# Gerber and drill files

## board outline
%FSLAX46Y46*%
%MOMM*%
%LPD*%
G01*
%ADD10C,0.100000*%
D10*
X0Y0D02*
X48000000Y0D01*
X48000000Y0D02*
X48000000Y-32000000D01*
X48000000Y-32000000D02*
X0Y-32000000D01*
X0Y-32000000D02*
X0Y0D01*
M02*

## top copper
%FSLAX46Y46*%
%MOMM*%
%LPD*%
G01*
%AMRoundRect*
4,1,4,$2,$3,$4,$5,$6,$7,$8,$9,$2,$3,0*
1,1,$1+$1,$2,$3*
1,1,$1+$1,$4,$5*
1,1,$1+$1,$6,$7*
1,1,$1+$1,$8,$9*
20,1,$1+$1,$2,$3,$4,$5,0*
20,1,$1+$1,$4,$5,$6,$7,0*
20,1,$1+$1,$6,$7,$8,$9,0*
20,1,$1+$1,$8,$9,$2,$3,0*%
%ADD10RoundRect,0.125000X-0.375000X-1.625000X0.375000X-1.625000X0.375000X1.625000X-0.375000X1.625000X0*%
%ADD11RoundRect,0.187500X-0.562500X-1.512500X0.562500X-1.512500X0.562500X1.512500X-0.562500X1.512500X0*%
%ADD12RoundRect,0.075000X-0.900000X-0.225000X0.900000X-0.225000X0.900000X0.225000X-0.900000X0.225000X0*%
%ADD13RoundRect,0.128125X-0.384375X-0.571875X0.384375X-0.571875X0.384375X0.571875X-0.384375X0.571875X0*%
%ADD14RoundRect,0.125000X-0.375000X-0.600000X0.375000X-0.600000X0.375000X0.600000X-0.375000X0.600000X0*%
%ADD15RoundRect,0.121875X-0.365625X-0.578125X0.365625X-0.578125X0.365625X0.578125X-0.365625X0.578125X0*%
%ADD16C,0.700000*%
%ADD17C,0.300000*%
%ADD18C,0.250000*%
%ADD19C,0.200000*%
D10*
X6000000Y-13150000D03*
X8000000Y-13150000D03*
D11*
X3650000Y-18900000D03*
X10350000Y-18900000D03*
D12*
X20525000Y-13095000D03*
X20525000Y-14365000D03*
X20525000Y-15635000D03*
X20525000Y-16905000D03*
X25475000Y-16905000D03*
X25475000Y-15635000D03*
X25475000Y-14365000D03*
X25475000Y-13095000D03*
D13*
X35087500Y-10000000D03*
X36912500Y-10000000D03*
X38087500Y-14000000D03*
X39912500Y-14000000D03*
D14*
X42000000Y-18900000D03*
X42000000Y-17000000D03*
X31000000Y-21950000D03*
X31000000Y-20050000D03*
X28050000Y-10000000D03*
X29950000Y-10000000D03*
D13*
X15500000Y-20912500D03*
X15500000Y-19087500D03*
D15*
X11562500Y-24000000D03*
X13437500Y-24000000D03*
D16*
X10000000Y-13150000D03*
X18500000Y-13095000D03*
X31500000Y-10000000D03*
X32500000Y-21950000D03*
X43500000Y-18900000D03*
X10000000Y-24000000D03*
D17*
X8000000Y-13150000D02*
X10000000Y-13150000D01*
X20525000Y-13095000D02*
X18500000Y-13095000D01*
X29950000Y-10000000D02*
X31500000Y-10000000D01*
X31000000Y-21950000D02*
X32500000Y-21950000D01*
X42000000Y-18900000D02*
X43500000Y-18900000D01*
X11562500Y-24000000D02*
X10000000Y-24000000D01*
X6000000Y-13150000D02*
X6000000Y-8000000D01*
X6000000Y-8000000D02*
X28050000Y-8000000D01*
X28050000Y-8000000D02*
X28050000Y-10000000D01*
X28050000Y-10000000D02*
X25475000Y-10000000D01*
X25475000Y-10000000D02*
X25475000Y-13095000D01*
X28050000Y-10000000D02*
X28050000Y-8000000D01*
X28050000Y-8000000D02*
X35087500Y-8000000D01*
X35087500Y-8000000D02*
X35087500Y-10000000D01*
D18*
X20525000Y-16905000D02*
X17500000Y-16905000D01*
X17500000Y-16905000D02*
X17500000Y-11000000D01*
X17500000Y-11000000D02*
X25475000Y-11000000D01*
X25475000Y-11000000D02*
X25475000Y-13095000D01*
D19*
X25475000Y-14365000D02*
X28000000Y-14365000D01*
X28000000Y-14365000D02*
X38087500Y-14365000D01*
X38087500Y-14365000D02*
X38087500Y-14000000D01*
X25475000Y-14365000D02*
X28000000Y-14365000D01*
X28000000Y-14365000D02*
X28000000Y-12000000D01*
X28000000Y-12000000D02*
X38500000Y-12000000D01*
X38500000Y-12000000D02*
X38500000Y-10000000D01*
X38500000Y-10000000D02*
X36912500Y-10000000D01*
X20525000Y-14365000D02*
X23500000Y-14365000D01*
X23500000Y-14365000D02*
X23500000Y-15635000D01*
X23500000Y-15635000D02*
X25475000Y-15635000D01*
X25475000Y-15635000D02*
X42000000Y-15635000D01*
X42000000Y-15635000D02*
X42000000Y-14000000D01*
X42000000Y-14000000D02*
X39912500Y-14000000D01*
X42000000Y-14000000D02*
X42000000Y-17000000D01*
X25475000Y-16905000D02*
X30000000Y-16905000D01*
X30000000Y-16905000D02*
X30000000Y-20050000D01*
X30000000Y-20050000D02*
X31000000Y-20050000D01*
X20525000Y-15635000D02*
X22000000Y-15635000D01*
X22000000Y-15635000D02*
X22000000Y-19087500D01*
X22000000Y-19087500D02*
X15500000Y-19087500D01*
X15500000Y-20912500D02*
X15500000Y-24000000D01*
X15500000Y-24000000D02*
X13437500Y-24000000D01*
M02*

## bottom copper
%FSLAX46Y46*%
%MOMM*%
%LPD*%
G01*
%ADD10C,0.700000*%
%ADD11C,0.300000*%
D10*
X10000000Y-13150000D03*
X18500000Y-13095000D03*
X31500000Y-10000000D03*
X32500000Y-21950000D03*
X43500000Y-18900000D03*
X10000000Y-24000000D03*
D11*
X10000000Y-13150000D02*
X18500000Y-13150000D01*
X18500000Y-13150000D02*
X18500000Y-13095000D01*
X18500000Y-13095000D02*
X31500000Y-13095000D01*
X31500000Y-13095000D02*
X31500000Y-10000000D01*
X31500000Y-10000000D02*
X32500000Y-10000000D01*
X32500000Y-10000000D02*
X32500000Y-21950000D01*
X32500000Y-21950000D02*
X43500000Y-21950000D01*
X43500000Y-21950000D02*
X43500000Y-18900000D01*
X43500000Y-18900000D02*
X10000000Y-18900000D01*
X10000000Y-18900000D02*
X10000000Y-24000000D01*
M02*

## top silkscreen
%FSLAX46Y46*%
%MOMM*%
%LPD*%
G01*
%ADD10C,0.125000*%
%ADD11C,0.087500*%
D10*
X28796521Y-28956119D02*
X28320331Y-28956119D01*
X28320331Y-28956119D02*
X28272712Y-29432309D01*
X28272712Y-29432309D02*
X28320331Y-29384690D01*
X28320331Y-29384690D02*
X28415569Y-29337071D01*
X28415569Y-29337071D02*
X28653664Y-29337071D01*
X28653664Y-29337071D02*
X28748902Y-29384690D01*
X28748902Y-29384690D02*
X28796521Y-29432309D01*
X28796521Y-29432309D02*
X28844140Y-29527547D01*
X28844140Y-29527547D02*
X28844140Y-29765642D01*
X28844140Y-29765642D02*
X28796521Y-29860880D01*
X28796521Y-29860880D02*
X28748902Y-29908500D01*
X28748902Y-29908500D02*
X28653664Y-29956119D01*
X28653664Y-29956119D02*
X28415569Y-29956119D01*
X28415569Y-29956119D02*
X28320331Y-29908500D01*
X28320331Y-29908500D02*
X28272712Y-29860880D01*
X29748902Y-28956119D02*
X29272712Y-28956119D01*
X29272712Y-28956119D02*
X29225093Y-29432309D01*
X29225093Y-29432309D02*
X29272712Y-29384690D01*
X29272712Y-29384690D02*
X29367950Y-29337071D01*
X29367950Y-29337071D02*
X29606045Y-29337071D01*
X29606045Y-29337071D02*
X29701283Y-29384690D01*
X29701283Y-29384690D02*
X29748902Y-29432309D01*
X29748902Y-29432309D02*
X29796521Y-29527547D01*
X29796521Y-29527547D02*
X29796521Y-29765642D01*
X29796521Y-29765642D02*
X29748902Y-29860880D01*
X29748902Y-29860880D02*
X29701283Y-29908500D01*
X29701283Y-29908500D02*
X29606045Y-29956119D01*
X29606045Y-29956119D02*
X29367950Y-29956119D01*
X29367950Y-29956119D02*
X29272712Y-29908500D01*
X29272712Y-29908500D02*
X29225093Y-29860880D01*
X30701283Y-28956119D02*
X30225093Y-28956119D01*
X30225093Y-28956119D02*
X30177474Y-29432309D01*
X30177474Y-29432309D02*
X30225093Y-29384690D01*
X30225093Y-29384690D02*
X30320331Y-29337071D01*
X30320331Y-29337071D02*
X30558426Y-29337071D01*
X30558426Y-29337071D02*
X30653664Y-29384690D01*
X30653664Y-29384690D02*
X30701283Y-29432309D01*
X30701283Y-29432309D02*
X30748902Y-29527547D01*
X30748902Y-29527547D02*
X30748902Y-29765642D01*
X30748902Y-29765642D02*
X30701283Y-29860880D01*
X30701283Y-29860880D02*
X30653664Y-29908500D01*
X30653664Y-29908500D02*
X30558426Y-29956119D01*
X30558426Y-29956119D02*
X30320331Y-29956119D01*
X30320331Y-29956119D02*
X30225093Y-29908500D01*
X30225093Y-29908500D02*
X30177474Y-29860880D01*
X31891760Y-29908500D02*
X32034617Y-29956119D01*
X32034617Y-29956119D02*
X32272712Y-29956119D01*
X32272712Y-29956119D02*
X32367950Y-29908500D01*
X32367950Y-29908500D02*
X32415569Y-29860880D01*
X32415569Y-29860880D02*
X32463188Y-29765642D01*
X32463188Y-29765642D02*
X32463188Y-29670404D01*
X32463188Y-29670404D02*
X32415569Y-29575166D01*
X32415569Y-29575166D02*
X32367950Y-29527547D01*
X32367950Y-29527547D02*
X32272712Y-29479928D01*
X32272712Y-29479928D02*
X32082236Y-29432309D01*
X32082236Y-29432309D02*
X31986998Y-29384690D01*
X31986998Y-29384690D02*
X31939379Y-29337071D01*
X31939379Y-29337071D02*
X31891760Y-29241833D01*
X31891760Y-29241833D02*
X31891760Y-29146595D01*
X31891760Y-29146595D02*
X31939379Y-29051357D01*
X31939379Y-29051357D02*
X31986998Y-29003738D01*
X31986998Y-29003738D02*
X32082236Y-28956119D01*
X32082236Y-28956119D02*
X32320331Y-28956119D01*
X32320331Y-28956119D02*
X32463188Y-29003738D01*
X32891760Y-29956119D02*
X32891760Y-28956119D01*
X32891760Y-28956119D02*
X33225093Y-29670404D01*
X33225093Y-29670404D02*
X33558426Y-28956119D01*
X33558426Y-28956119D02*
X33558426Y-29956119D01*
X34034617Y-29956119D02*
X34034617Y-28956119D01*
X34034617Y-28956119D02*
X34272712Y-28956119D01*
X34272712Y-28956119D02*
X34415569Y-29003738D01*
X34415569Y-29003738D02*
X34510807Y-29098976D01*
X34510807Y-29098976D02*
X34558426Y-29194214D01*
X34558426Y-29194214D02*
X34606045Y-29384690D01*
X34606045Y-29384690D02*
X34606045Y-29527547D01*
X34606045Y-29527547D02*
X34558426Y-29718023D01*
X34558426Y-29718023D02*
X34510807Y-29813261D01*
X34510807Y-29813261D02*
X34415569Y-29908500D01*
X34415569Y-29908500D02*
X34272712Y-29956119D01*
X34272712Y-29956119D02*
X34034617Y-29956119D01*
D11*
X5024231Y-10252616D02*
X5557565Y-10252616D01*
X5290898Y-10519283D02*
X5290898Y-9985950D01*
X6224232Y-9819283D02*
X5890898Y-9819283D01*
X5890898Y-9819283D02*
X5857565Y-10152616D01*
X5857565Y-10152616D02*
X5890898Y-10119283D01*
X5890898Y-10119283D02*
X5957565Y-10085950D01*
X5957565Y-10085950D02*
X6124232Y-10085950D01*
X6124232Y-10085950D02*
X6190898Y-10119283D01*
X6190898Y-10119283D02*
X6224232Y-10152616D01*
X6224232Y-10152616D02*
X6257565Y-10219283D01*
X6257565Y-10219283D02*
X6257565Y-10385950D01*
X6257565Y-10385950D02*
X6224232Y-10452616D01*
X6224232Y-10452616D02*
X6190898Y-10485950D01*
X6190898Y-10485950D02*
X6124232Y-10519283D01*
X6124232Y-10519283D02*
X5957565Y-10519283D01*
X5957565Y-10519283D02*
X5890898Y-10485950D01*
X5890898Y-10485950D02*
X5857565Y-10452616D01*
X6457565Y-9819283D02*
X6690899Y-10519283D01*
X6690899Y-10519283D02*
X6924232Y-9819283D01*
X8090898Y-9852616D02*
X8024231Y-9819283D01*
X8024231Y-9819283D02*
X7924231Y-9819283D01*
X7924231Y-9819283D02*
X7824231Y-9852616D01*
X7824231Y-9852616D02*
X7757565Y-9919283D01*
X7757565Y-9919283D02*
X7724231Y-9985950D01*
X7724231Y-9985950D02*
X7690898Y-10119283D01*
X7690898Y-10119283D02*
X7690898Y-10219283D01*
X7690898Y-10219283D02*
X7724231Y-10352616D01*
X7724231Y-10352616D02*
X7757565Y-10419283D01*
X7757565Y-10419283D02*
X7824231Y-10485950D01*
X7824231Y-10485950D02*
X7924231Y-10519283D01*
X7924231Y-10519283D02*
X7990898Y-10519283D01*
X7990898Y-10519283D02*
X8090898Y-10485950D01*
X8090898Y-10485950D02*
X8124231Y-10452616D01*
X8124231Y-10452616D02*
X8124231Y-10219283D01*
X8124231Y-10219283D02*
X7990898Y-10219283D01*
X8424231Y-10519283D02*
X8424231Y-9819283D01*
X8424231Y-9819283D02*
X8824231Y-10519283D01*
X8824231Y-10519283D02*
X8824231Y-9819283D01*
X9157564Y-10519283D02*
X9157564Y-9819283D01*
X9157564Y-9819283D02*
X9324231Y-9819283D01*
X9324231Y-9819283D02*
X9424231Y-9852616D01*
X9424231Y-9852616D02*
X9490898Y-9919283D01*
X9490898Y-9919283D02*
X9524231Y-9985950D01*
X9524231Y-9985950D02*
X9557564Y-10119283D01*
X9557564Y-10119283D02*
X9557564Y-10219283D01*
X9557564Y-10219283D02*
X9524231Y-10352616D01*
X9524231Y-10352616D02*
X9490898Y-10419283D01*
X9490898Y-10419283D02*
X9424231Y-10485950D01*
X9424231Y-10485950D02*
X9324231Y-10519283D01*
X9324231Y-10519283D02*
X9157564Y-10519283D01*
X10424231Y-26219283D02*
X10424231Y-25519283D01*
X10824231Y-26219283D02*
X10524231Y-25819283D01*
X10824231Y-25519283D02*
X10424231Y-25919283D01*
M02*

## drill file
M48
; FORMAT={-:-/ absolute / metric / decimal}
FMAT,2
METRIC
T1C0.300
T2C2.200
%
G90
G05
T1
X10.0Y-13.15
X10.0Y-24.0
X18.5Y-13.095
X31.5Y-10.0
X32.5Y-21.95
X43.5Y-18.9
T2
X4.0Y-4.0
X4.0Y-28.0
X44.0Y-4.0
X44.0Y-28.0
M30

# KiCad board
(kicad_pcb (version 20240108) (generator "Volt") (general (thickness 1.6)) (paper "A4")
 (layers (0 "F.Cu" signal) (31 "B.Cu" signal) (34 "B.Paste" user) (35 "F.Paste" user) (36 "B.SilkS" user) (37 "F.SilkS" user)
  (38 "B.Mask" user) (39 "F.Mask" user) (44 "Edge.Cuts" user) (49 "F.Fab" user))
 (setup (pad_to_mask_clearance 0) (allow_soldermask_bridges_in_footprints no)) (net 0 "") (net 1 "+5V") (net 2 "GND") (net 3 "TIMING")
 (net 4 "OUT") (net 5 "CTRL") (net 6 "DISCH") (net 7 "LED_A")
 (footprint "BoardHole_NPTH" (layer "F.Cu") (at 4 4)
  (pad "" np_thru_hole circle (at 0 0) (size 2.2 2.2) (drill 2.2) (layers "*.Cu" "*.Mask")))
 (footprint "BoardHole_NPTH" (layer "F.Cu") (at 44 4)
  (pad "" np_thru_hole circle (at 0 0) (size 2.2 2.2) (drill 2.2) (layers "*.Cu" "*.Mask")))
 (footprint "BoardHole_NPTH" (layer "F.Cu") (at 4 28)
  (pad "" np_thru_hole circle (at 0 0) (size 2.2 2.2) (drill 2.2) (layers "*.Cu" "*.Mask")))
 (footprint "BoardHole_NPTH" (layer "F.Cu") (at 44 28)
  (pad "" np_thru_hole circle (at 0 0) (size 2.2 2.2) (drill 2.2) (layers "*.Cu" "*.Mask")))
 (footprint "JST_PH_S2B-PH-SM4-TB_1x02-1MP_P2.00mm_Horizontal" (layer "F.Cu") (at 7 16)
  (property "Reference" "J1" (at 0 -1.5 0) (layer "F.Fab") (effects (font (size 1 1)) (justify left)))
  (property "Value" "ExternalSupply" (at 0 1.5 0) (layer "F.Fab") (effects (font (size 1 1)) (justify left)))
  (pad "1" smd roundrect (at -1 -2.85) (size 1 3.5) (layers "F.Cu" "F.Paste" "F.Mask") (roundrect_rratio 0.125) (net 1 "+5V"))
  (pad "2" smd roundrect (at 1 -2.85) (size 1 3.5) (layers "F.Cu" "F.Paste" "F.Mask") (roundrect_rratio 0.125) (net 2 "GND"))
  (pad "MP1" smd roundrect (at -3.35 2.9) (size 1.5 3.4) (layers "F.Cu" "F.Paste" "F.Mask") (roundrect_rratio 0.125))
  (pad "MP2" smd roundrect (at 3.35 2.9) (size 1.5 3.4) (layers "F.Cu" "F.Paste" "F.Mask") (roundrect_rratio 0.125)))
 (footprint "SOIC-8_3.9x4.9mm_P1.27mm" (layer "F.Cu") (at 23 15)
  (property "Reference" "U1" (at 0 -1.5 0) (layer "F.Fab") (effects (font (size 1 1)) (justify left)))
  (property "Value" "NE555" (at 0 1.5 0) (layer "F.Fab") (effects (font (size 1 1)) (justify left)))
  (pad "1" smd roundrect (at -2.475 -1.905) (size 1.95 0.6) (layers "F.Cu" "F.Paste" "F.Mask") (roundrect_rratio 0.125) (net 2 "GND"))
  (pad "2" smd roundrect (at -2.475 -0.635) (size 1.95 0.6) (layers "F.Cu" "F.Paste" "F.Mask") (roundrect_rratio 0.125) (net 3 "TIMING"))
  (pad "3" smd roundrect (at -2.475 0.635) (size 1.95 0.6) (layers "F.Cu" "F.Paste" "F.Mask") (roundrect_rratio 0.125) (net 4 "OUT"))
  (pad "4" smd roundrect (at -2.475 1.905) (size 1.95 0.6) (layers "F.Cu" "F.Paste" "F.Mask") (roundrect_rratio 0.125) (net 1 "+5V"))
  (pad "5" smd roundrect (at 2.475 1.905) (size 1.95 0.6) (layers "F.Cu" "F.Paste" "F.Mask") (roundrect_rratio 0.125) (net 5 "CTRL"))
  (pad "6" smd roundrect (at 2.475 0.635) (size 1.95 0.6) (layers "F.Cu" "F.Paste" "F.Mask") (roundrect_rratio 0.125) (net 3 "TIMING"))
  (pad "7" smd roundrect (at 2.475 -0.635) (size 1.95 0.6) (layers "F.Cu" "F.Paste" "F.Mask") (roundrect_rratio 0.125) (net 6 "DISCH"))
  (pad "8" smd roundrect (at 2.475 -1.905) (size 1.95 0.6) (layers "F.Cu" "F.Paste" "F.Mask") (roundrect_rratio 0.125) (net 1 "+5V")))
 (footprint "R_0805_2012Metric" (layer "F.Cu") (at 36 10)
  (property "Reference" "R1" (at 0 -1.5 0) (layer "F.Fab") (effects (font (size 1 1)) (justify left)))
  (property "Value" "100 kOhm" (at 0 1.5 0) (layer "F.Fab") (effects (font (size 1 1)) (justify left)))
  (pad "1" smd roundrect (at -0.9125 0) (size 1.025 1.4) (layers "F.Cu" "F.Paste" "F.Mask") (roundrect_rratio 0.125) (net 1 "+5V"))
  (pad "2" smd roundrect (at 0.9125 0) (size 1.025 1.4) (layers "F.Cu" "F.Paste" "F.Mask") (roundrect_rratio 0.125) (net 6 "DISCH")))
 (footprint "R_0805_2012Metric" (layer "F.Cu") (at 39 14)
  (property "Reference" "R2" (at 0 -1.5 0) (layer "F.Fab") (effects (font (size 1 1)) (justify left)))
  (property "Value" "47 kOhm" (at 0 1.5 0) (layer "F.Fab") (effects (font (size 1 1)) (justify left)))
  (pad "1" smd roundrect (at -0.9125 0) (size 1.025 1.4) (layers "F.Cu" "F.Paste" "F.Mask") (roundrect_rratio 0.125) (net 6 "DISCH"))
  (pad "2" smd roundrect (at 0.9125 0) (size 1.025 1.4) (layers "F.Cu" "F.Paste" "F.Mask") (roundrect_rratio 0.125) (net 3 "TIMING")))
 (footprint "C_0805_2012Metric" (layer "F.Cu") (at 42 17.95 90)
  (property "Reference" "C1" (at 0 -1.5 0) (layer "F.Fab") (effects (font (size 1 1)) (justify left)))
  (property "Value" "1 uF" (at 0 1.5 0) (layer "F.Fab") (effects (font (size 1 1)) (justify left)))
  (pad "1" smd roundrect (at -0.95 0) (size 1 1.45) (layers "F.Cu" "F.Paste" "F.Mask") (roundrect_rratio 0.125) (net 3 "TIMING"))
  (pad "2" smd roundrect (at 0.95 0) (size 1 1.45) (layers "F.Cu" "F.Paste" "F.Mask") (roundrect_rratio 0.125) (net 2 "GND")))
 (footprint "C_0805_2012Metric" (layer "F.Cu") (at 31 21 90)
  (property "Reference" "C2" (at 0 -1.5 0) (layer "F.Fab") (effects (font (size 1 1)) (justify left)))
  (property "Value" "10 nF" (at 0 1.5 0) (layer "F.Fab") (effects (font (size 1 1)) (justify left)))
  (pad "1" smd roundrect (at -0.95 0) (size 1 1.45) (layers "F.Cu" "F.Paste" "F.Mask") (roundrect_rratio 0.125) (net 5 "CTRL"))
  (pad "2" smd roundrect (at 0.95 0) (size 1 1.45) (layers "F.Cu" "F.Paste" "F.Mask") (roundrect_rratio 0.125) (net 2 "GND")))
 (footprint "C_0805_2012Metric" (layer "F.Cu") (at 29 10)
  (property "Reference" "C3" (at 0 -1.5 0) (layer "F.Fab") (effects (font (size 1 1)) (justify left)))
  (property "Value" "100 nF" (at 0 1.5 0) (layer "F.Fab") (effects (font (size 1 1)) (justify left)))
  (pad "1" smd roundrect (at -0.95 0) (size 1 1.45) (layers "F.Cu" "F.Paste" "F.Mask") (roundrect_rratio 0.125) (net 1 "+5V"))
  (pad "2" smd roundrect (at 0.95 0) (size 1 1.45) (layers "F.Cu" "F.Paste" "F.Mask") (roundrect_rratio 0.125) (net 2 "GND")))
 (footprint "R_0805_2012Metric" (layer "F.Cu") (at 15.5 20 90)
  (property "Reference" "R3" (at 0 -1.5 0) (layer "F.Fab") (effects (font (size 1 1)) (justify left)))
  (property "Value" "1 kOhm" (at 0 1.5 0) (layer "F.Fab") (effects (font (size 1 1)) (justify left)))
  (pad "1" smd roundrect (at -0.9125 0) (size 1.025 1.4) (layers "F.Cu" "F.Paste" "F.Mask") (roundrect_rratio 0.125) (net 4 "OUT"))
  (pad "2" smd roundrect (at 0.9125 0) (size 1.025 1.4) (layers "F.Cu" "F.Paste" "F.Mask") (roundrect_rratio 0.125) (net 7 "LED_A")))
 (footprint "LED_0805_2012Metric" (layer "F.Cu") (at 12.5 24)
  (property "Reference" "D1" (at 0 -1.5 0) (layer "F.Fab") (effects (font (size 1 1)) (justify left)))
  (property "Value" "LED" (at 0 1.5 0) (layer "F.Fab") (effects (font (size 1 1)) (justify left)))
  (pad "1" smd roundrect (at -0.9375 0) (size 0.975 1.4) (layers "F.Cu" "F.Paste" "F.Mask") (roundrect_rratio 0.125) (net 2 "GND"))
  (pad "2" smd roundrect (at 0.9375 0) (size 0.975 1.4) (layers "F.Cu" "F.Paste" "F.Mask") (roundrect_rratio 0.125) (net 7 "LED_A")))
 (segment (start 8 13.15) (end 10 13.15) (width 0.3) (layer "F.Cu") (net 2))
 (segment (start 20.525 13.095) (end 18.5 13.095) (width 0.3) (layer "F.Cu") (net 2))
 (segment (start 29.95 10) (end 31.5 10) (width 0.3) (layer "F.Cu") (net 2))
 (segment (start 31 21.95) (end 32.5 21.95) (width 0.3) (layer "F.Cu") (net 2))
 (segment (start 42 18.9) (end 43.5 18.9) (width 0.3) (layer "F.Cu") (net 2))
 (segment (start 11.5625 24) (end 10 24) (width 0.3) (layer "F.Cu") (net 2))
 (segment (start 10 13.15) (end 18.5 13.15) (width 0.3) (layer "B.Cu") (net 2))
 (segment (start 18.5 13.15) (end 18.5 13.095) (width 0.3) (layer "B.Cu") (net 2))
 (segment (start 18.5 13.095) (end 31.5 13.095) (width 0.3) (layer "B.Cu") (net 2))
 (segment (start 31.5 13.095) (end 31.5 10) (width 0.3) (layer "B.Cu") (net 2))
 (segment (start 31.5 10) (end 32.5 10) (width 0.3) (layer "B.Cu") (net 2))
 (segment (start 32.5 10) (end 32.5 21.95) (width 0.3) (layer "B.Cu") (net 2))
 (segment (start 32.5 21.95) (end 43.5 21.95) (width 0.3) (layer "B.Cu") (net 2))
 (segment (start 43.5 21.95) (end 43.5 18.9) (width 0.3) (layer "B.Cu") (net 2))
 (segment (start 43.5 18.9) (end 10 18.9) (width 0.3) (layer "B.Cu") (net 2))
 (segment (start 10 18.9) (end 10 24) (width 0.3) (layer "B.Cu") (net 2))
 (segment (start 6 13.15) (end 6 8) (width 0.3) (layer "F.Cu") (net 1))
 (segment (start 6 8) (end 28.05 8) (width 0.3) (layer "F.Cu") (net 1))
 (segment (start 28.05 8) (end 28.05 10) (width 0.3) (layer "F.Cu") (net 1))
 (segment (start 28.05 10) (end 25.475 10) (width 0.3) (layer "F.Cu") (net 1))
 (segment (start 25.475 10) (end 25.475 13.095) (width 0.3) (layer "F.Cu") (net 1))
 (segment (start 28.05 10) (end 28.05 8) (width 0.3) (layer "F.Cu") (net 1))
 (segment (start 28.05 8) (end 35.0875 8) (width 0.3) (layer "F.Cu") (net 1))
 (segment (start 35.0875 8) (end 35.0875 10) (width 0.3) (layer "F.Cu") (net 1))
 (segment (start 20.525 16.905) (end 17.5 16.905) (width 0.25) (layer "F.Cu") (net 1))
 (segment (start 17.5 16.905) (end 17.5 11) (width 0.25) (layer "F.Cu") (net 1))
 (segment (start 17.5 11) (end 25.475 11) (width 0.25) (layer "F.Cu") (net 1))
 (segment (start 25.475 11) (end 25.475 13.095) (width 0.25) (layer "F.Cu") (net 1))
 (segment (start 25.475 14.365) (end 28 14.365) (width 0.2) (layer "F.Cu") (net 6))
 (segment (start 28 14.365) (end 38.0875 14.365) (width 0.2) (layer "F.Cu") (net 6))
 (segment (start 38.0875 14.365) (end 38.0875 14) (width 0.2) (layer "F.Cu") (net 6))
 (segment (start 25.475 14.365) (end 28 14.365) (width 0.2) (layer "F.Cu") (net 6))
 (segment (start 28 14.365) (end 28 12) (width 0.2) (layer "F.Cu") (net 6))
 (segment (start 28 12) (end 38.5 12) (width 0.2) (layer "F.Cu") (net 6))
 (segment (start 38.5 12) (end 38.5 10) (width 0.2) (layer "F.Cu") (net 6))
 (segment (start 38.5 10) (end 36.9125 10) (width 0.2) (layer "F.Cu") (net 6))
 (segment (start 20.525 14.365) (end 23.5 14.365) (width 0.2) (layer "F.Cu") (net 3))
 (segment (start 23.5 14.365) (end 23.5 15.635) (width 0.2) (layer "F.Cu") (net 3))
 (segment (start 23.5 15.635) (end 25.475 15.635) (width 0.2) (layer "F.Cu") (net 3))
 (segment (start 25.475 15.635) (end 42 15.635) (width 0.2) (layer "F.Cu") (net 3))
 (segment (start 42 15.635) (end 42 14) (width 0.2) (layer "F.Cu") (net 3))
 (segment (start 42 14) (end 39.9125 14) (width 0.2) (layer "F.Cu") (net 3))
 (segment (start 42 14) (end 42 17) (width 0.2) (layer "F.Cu") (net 3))
 (segment (start 25.475 16.905) (end 30 16.905) (width 0.2) (layer "F.Cu") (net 5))
 (segment (start 30 16.905) (end 30 20.05) (width 0.2) (layer "F.Cu") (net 5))
 (segment (start 30 20.05) (end 31 20.05) (width 0.2) (layer "F.Cu") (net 5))
 (segment (start 20.525 15.635) (end 22 15.635) (width 0.2) (layer "F.Cu") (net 4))
 (segment (start 22 15.635) (end 22 19.0875) (width 0.2) (layer "F.Cu") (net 4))
 (segment (start 22 19.0875) (end 15.5 19.0875) (width 0.2) (layer "F.Cu") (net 4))
 (segment (start 15.5 20.9125) (end 15.5 24) (width 0.2) (layer "F.Cu") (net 7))
 (segment (start 15.5 24) (end 13.4375 24) (width 0.2) (layer "F.Cu") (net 7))
 (via (at 10 13.15) (size 0.7) (drill 0.3) (layers "F.Cu" "B.Cu") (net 2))
 (via (at 18.5 13.095) (size 0.7) (drill 0.3) (layers "F.Cu" "B.Cu") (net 2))
 (via (at 31.5 10) (size 0.7) (drill 0.3) (layers "F.Cu" "B.Cu") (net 2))
 (via (at 32.5 21.95) (size 0.7) (drill 0.3) (layers "F.Cu" "B.Cu") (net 2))
 (via (at 43.5 18.9) (size 0.7) (drill 0.3) (layers "F.Cu" "B.Cu") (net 2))
 (via (at 10 24) (size 0.7) (drill 0.3) (layers "F.Cu" "B.Cu") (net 2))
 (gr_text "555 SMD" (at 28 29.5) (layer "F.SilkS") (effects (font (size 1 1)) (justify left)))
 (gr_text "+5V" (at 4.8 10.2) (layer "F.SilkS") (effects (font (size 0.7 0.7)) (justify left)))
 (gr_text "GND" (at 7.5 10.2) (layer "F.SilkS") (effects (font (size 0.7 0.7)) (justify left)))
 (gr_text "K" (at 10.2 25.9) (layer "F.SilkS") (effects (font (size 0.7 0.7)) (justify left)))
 (gr_line (start 0 0) (end 48 0) (stroke (width 0.1) (type default)) (layer "Edge.Cuts"))
 (gr_line (start 48 0) (end 48 32) (stroke (width 0.1) (type default)) (layer "Edge.Cuts"))
 (gr_line (start 48 32) (end 0 32) (stroke (width 0.1) (type default)) (layer "Edge.Cuts"))
 (gr_line (start 0 32) (end 0 0) (stroke (width 0.1) (type default)) (layer "Edge.Cuts")))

